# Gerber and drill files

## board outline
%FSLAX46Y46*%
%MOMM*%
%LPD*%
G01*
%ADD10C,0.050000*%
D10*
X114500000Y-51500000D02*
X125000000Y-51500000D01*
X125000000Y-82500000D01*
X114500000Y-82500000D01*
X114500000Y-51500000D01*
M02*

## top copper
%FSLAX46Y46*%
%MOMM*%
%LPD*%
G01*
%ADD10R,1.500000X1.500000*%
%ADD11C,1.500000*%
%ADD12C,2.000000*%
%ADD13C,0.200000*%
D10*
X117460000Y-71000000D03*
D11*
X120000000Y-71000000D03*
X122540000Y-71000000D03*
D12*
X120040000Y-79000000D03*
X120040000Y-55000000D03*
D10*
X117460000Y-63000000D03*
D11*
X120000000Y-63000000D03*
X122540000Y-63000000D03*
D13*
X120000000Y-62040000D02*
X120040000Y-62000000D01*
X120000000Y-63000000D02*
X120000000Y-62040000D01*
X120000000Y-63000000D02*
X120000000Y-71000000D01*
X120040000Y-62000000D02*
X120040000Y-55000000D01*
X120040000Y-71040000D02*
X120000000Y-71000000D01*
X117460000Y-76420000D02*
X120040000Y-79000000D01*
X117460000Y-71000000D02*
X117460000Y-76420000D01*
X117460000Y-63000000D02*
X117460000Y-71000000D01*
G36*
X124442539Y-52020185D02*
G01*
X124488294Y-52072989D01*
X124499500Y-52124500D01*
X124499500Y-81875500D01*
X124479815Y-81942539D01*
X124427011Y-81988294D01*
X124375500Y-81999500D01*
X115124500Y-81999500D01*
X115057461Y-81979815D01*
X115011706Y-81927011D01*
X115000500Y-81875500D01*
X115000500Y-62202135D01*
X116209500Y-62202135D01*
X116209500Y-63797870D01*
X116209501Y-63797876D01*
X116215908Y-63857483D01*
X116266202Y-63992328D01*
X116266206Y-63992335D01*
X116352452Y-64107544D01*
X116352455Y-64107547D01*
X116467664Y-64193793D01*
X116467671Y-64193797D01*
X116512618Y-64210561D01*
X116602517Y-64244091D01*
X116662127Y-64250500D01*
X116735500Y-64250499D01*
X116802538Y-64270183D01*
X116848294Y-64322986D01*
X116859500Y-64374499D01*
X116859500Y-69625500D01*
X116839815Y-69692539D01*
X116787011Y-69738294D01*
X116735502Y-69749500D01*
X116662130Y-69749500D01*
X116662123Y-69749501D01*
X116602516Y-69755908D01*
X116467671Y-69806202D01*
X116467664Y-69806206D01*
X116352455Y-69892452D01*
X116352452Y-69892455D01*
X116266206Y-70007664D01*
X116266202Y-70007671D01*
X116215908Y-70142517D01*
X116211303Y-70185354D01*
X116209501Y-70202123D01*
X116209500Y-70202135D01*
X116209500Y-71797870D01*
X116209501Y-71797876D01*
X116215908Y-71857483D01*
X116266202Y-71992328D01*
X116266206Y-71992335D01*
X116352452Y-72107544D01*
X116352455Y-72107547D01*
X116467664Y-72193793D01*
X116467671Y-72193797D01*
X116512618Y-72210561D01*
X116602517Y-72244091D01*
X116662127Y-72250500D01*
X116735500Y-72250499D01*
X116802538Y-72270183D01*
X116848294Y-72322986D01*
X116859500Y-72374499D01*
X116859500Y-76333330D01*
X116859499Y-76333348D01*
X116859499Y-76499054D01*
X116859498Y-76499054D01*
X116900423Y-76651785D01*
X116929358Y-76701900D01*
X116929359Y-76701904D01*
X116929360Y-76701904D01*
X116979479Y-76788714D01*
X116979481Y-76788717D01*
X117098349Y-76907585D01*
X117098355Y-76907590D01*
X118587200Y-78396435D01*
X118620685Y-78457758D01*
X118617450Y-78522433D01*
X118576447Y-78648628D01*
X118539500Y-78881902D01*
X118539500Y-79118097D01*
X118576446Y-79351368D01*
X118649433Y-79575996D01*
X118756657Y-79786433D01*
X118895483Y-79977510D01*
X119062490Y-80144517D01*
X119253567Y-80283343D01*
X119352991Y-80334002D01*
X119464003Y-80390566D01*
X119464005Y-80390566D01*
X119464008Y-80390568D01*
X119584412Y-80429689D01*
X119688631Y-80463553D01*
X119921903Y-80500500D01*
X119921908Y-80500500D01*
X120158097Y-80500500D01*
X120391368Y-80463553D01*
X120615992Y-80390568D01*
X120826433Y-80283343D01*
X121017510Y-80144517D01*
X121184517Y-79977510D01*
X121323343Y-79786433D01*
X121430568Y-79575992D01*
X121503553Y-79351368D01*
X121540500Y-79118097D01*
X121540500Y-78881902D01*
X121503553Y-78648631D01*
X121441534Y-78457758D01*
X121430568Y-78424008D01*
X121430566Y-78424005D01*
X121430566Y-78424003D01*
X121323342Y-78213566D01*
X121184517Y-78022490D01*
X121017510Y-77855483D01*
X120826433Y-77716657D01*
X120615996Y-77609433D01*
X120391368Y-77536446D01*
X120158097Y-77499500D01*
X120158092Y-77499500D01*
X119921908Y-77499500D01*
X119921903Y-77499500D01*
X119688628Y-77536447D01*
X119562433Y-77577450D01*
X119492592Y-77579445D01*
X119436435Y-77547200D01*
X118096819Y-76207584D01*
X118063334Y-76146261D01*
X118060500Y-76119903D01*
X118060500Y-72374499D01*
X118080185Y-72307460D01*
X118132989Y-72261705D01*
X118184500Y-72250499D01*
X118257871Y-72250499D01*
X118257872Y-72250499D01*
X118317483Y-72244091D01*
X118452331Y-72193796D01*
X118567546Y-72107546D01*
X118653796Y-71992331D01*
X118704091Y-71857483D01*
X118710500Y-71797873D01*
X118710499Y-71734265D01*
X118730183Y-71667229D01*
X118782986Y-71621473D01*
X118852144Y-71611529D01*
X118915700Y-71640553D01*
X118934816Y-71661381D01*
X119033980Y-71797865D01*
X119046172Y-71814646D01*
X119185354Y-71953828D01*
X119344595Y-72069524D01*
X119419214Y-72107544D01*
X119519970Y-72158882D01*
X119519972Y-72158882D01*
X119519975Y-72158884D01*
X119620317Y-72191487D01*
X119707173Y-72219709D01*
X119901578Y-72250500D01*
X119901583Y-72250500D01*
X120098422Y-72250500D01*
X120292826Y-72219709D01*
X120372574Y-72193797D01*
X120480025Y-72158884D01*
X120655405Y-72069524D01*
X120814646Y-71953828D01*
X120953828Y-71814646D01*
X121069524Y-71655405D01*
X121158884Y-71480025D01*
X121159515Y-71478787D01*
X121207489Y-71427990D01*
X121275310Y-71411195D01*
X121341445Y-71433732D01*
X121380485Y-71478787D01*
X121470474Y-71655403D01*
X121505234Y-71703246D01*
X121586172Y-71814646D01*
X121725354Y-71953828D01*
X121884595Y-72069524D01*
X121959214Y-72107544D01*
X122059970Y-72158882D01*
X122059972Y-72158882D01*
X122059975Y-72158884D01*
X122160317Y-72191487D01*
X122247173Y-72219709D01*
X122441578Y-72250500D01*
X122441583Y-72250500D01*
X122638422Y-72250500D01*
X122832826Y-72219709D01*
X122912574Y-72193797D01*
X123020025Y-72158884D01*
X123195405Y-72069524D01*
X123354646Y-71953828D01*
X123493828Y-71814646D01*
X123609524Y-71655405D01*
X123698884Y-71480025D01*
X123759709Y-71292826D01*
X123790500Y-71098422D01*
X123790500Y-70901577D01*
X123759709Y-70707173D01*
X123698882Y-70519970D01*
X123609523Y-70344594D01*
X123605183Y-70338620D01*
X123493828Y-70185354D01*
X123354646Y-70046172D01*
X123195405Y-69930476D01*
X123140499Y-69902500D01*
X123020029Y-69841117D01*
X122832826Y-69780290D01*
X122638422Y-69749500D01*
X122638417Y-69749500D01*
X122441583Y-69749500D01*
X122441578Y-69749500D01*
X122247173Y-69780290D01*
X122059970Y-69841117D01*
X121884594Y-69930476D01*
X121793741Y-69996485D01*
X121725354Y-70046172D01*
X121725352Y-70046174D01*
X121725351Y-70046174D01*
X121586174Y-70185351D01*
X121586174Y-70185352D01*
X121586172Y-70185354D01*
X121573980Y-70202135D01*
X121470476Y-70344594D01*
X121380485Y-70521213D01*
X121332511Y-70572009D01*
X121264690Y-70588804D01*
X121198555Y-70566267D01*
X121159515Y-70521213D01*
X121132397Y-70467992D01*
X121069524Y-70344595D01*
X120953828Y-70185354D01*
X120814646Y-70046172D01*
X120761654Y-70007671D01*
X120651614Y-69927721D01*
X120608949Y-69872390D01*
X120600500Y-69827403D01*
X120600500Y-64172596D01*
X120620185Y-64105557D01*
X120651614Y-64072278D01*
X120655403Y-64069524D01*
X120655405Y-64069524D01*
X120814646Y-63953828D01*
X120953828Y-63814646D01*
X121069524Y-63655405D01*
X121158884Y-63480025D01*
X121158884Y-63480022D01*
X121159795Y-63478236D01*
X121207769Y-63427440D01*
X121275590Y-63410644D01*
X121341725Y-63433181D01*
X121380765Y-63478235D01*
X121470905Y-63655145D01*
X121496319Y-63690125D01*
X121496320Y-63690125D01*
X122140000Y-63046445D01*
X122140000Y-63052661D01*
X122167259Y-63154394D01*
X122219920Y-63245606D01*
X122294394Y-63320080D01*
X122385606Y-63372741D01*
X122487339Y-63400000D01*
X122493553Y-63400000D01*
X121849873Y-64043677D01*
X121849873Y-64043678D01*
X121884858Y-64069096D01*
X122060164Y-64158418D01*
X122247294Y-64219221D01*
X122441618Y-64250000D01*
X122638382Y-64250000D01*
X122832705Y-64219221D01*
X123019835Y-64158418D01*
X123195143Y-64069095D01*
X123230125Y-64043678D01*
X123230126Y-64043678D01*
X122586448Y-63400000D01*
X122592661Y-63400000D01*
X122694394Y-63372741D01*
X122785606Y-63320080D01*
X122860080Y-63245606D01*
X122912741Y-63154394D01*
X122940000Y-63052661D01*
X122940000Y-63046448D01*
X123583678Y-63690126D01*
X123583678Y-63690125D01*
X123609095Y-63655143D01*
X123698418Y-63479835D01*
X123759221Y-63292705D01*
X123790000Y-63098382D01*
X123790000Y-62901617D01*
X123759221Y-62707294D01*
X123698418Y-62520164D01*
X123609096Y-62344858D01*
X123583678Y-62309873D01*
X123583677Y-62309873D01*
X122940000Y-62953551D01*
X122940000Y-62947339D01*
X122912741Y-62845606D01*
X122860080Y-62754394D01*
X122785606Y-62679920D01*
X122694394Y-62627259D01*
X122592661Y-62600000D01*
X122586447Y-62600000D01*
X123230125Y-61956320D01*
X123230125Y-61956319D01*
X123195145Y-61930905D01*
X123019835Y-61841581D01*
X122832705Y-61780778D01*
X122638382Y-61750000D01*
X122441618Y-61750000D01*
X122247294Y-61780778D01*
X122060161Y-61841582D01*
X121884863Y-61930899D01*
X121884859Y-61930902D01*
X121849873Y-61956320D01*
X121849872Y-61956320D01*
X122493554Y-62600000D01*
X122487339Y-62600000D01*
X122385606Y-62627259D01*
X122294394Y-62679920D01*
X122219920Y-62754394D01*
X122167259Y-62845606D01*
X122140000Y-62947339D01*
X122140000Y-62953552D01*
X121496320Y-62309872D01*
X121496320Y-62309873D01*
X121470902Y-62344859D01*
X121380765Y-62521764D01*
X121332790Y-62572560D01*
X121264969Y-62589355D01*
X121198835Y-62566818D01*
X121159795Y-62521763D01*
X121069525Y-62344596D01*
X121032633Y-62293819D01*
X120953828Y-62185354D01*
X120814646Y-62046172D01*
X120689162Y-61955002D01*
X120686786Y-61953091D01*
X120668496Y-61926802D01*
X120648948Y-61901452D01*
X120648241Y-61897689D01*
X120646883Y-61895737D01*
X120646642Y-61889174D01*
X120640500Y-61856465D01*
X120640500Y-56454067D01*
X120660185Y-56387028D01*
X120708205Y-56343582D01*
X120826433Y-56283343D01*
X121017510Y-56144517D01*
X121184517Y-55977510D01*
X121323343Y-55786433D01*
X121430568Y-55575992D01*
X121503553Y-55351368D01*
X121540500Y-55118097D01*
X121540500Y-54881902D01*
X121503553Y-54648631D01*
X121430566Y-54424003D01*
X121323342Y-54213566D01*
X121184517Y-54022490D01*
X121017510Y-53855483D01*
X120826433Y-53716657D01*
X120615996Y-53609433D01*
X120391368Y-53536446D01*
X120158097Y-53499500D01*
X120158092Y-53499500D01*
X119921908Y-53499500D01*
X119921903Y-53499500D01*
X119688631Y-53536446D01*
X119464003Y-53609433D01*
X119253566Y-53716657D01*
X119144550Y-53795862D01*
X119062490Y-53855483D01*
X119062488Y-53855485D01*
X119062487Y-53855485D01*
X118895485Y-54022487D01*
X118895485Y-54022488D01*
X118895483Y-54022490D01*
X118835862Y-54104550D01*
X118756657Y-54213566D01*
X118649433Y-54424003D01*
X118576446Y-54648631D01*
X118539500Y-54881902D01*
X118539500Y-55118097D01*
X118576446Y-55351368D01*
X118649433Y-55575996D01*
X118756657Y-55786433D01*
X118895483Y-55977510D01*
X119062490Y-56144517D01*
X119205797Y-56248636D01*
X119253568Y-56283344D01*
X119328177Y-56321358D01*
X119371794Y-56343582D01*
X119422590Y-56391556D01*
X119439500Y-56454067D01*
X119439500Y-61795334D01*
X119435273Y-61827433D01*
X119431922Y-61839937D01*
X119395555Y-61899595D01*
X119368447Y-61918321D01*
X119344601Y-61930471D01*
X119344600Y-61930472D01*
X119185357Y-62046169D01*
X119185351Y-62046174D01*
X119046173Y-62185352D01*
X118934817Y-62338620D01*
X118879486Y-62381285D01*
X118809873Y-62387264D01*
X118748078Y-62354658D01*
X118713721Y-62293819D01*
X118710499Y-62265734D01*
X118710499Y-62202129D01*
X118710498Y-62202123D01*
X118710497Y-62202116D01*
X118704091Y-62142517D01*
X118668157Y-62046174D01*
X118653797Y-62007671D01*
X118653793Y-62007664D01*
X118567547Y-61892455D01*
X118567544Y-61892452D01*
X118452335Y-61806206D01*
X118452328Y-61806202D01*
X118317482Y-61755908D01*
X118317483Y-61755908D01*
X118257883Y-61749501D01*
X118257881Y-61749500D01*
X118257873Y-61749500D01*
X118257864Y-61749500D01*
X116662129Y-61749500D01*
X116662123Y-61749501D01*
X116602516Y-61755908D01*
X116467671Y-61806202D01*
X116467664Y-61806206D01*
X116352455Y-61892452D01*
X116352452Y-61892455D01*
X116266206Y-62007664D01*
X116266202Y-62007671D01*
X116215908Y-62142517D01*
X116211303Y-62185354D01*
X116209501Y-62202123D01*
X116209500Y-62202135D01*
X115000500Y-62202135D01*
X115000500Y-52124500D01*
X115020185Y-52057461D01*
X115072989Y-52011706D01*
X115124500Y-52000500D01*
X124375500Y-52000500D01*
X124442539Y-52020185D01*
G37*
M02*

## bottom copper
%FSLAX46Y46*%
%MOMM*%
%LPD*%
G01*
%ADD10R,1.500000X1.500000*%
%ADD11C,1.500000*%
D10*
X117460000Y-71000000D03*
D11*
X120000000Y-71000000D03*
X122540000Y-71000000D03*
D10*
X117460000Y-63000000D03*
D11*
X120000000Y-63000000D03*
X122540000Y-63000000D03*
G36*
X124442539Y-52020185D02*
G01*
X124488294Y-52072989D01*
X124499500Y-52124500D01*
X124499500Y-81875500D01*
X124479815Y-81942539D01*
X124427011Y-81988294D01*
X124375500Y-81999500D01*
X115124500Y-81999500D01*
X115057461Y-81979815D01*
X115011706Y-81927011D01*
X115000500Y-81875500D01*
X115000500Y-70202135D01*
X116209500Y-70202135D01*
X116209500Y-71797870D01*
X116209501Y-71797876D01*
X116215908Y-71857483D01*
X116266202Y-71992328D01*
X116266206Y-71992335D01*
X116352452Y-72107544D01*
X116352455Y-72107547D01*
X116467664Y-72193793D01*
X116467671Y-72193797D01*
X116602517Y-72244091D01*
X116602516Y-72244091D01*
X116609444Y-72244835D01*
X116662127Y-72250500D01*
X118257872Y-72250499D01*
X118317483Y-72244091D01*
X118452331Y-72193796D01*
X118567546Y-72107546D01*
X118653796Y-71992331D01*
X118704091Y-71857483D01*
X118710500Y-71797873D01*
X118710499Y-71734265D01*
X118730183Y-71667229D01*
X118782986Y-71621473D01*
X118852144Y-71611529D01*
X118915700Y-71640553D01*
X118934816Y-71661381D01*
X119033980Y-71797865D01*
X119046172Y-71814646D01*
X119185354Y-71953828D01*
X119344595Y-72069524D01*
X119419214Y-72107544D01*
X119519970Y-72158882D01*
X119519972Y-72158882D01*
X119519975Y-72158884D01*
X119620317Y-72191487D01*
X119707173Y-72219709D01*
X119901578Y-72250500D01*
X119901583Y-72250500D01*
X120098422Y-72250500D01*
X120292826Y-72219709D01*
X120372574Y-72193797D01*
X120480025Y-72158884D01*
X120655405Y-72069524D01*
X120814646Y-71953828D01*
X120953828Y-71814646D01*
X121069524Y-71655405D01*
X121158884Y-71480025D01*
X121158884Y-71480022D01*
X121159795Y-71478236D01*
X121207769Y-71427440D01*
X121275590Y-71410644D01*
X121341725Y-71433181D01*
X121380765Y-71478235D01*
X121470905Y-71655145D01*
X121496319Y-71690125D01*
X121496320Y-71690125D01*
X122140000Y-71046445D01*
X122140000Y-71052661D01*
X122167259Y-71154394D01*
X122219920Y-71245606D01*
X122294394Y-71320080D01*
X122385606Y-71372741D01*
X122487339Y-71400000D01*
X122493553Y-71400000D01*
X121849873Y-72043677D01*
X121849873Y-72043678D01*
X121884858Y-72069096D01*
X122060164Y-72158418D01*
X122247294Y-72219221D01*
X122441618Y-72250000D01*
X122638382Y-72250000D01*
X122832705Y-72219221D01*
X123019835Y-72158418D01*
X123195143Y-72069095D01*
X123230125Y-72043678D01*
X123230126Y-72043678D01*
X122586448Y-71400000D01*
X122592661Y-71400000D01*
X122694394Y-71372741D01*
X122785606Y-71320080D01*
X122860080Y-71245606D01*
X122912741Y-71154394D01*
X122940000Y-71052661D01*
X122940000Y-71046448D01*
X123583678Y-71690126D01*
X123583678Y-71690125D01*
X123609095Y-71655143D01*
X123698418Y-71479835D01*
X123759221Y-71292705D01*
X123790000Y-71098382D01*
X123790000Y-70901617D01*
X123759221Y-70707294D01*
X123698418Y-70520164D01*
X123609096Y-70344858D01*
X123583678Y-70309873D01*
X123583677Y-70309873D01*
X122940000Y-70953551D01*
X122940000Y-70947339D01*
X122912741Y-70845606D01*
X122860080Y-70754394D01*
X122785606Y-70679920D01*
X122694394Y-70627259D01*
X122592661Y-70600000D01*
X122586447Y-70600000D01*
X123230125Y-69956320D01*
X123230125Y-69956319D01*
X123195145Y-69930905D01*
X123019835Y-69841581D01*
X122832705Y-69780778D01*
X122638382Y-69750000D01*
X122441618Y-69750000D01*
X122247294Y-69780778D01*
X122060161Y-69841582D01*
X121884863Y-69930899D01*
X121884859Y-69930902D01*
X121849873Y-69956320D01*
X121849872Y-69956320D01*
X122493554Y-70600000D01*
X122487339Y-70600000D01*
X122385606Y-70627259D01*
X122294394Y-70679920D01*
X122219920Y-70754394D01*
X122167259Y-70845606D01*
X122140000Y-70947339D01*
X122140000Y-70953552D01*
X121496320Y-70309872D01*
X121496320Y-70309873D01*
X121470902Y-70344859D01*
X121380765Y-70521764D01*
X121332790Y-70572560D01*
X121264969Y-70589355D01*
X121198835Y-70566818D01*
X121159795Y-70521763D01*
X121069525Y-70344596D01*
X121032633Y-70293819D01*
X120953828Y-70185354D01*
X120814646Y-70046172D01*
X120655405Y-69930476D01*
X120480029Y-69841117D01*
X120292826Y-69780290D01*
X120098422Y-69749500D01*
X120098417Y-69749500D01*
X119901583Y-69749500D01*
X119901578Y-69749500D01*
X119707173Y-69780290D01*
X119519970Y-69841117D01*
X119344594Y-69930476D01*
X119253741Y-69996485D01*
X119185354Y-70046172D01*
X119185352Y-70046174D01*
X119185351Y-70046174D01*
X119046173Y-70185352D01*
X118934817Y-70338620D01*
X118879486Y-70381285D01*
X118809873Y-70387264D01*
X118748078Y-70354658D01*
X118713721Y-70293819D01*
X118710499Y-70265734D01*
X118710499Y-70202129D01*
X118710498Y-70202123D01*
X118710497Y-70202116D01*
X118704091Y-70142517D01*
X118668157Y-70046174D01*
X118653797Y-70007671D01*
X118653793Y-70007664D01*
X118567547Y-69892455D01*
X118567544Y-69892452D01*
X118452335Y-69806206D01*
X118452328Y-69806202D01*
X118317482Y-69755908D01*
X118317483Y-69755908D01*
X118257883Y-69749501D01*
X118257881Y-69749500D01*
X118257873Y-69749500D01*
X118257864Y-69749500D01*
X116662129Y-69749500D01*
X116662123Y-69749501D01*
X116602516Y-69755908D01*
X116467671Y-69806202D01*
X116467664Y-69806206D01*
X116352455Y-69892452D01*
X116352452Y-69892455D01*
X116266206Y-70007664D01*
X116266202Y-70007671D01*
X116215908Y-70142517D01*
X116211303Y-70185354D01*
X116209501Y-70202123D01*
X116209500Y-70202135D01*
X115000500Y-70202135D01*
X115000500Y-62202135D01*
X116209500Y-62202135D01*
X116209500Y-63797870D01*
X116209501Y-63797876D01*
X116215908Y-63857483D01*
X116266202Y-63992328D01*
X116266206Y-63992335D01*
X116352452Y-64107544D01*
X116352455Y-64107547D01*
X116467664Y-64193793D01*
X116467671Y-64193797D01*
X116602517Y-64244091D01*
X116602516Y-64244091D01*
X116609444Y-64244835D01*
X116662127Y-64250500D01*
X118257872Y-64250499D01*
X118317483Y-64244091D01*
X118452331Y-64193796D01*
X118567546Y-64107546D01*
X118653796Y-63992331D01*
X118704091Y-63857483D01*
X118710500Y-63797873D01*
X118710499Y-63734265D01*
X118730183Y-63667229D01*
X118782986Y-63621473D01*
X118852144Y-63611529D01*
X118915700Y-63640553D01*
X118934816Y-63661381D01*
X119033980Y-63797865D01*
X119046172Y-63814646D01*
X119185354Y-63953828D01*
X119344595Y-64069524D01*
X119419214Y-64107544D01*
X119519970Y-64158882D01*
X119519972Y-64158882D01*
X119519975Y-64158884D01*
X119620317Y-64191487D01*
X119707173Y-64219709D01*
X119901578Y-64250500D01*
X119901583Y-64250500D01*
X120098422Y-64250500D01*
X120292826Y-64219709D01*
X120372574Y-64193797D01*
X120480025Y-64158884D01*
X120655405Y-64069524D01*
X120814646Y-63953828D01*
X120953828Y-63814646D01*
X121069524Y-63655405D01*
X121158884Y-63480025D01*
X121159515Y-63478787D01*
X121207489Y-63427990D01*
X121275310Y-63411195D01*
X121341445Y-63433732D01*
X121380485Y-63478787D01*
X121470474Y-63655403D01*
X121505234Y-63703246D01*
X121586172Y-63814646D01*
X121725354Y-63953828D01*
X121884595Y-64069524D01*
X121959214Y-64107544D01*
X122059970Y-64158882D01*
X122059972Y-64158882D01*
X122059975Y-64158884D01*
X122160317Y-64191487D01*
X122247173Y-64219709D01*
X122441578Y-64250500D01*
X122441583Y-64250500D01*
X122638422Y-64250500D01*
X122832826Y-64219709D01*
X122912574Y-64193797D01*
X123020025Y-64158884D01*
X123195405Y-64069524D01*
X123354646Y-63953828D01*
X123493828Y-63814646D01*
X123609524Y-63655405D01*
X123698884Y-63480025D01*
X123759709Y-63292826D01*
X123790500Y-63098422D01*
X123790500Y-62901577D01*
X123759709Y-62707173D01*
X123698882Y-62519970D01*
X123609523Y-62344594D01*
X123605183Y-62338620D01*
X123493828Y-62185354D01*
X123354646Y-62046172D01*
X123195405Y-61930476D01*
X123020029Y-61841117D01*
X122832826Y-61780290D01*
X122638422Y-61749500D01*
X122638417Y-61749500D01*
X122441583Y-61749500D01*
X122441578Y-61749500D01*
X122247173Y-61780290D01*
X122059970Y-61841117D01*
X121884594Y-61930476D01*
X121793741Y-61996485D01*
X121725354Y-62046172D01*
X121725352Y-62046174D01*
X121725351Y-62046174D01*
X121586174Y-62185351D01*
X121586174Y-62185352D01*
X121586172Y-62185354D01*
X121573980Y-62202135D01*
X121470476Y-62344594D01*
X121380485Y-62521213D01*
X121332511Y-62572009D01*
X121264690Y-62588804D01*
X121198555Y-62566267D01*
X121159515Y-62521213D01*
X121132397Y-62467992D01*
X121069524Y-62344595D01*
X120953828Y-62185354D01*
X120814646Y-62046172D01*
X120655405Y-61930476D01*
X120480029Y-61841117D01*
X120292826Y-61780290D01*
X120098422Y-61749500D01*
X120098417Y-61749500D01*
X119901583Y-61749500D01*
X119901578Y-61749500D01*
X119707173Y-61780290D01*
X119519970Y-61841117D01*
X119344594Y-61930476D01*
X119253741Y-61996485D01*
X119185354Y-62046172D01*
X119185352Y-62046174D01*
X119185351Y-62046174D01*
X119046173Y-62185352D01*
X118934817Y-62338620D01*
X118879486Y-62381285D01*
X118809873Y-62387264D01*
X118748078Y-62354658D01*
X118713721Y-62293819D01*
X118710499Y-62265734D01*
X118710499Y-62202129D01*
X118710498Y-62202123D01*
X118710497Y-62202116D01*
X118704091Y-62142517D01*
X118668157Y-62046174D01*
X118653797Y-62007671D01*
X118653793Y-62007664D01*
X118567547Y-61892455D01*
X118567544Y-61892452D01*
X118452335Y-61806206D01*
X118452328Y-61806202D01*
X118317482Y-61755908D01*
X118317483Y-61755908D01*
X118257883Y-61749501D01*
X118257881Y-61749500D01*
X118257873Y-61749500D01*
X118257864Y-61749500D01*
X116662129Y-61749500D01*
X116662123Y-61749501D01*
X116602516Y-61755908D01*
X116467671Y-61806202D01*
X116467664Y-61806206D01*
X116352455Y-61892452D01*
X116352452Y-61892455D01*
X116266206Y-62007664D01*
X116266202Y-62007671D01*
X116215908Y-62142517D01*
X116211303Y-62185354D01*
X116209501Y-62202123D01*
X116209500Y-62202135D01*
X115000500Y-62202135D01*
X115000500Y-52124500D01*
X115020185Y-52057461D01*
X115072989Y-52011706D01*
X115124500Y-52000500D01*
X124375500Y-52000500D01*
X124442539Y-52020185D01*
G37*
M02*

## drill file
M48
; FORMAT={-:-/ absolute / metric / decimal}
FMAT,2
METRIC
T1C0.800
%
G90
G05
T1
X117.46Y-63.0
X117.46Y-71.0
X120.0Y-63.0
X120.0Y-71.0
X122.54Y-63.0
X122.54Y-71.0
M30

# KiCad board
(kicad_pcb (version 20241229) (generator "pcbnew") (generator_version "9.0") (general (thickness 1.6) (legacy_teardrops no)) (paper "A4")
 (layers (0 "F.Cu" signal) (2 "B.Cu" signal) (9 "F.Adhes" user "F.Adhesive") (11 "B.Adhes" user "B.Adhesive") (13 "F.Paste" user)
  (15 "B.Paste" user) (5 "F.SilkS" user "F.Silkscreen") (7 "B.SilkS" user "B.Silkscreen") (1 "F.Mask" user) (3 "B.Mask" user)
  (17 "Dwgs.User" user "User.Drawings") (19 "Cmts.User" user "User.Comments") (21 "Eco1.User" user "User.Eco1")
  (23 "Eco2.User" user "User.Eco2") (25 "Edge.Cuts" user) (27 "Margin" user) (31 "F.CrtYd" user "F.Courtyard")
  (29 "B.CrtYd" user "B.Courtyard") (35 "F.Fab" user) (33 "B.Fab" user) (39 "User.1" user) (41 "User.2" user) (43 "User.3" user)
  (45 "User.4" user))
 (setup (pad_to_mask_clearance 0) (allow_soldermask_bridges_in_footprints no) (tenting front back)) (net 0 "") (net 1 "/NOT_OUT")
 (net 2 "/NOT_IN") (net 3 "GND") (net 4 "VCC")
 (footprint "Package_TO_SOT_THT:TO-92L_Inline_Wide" (layer "F.Cu") (at 117.46 71)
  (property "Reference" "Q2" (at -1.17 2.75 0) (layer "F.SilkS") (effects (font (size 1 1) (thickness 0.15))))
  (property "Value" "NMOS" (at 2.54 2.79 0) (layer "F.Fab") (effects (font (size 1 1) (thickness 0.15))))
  (pad "1" thru_hole rect (at 0 0) (size 1.5 1.5) (drill 0.8) (layers "*.Cu" "*.Mask") (remove_unused_layers no) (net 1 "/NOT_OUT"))
  (pad "2" thru_hole circle (at 2.54 0) (size 1.5 1.5) (drill 0.8) (layers "*.Cu" "*.Mask") (remove_unused_layers no) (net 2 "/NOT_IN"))
  (pad "3" thru_hole circle (at 5.08 0) (size 1.5 1.5) (drill 0.8) (layers "*.Cu" "*.Mask") (remove_unused_layers no) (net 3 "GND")))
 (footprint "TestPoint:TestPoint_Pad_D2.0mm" (layer "F.Cu") (at 120.04 79)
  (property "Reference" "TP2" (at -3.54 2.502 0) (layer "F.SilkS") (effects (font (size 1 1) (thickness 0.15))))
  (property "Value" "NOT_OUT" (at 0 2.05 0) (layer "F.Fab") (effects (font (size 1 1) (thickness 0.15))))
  (pad "1" smd circle (at 0 0) (size 2 2) (layers "F.Cu" "F.Mask") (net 1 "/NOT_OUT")))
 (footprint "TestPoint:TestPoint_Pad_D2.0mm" (layer "F.Cu") (at 120.04 55)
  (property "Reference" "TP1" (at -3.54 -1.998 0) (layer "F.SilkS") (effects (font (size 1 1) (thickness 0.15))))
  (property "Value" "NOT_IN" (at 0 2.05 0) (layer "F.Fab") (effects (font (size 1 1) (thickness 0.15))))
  (pad "1" smd circle (at 0 0) (size 2 2) (layers "F.Cu" "F.Mask") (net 2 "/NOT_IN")))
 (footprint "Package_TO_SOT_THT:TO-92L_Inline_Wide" (layer "F.Cu") (at 117.46 63)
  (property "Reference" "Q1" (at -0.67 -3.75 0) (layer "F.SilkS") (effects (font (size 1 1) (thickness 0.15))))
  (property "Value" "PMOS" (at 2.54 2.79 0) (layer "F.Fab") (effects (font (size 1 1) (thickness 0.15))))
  (pad "1" thru_hole rect (at 0 0) (size 1.5 1.5) (drill 0.8) (layers "*.Cu" "*.Mask") (remove_unused_layers no) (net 1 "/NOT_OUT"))
  (pad "2" thru_hole circle (at 2.54 0) (size 1.5 1.5) (drill 0.8) (layers "*.Cu" "*.Mask") (remove_unused_layers no) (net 2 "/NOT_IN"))
  (pad "3" thru_hole circle (at 5.08 0) (size 1.5 1.5) (drill 0.8) (layers "*.Cu" "*.Mask") (remove_unused_layers no) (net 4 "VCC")))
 (gr_rect (start 114.5 51.5) (end 125 82.5) (stroke (width 0.05) (type default)) (fill no) (layer "Edge.Cuts"))
 (segment (start 120 62.04) (end 120.04 62) (width 0.2) (layer "F.Cu") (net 2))
 (segment (start 120 63) (end 120 62.04) (width 0.2) (layer "F.Cu") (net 2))
 (segment (start 120 63) (end 120 71) (width 0.2) (layer "F.Cu") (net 2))
 (segment (start 120.04 62) (end 120.04 55) (width 0.2) (layer "F.Cu") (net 2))
 (segment (start 120.04 71.04) (end 120 71) (width 0.2) (layer "F.Cu") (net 2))
 (segment (start 117.46 76.42) (end 120.04 79) (width 0.2) (layer "F.Cu") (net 1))
 (segment (start 117.46 71) (end 117.46 76.42) (width 0.2) (layer "F.Cu") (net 1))
 (segment (start 117.46 63) (end 117.46 71) (width 0.2) (layer "F.Cu") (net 1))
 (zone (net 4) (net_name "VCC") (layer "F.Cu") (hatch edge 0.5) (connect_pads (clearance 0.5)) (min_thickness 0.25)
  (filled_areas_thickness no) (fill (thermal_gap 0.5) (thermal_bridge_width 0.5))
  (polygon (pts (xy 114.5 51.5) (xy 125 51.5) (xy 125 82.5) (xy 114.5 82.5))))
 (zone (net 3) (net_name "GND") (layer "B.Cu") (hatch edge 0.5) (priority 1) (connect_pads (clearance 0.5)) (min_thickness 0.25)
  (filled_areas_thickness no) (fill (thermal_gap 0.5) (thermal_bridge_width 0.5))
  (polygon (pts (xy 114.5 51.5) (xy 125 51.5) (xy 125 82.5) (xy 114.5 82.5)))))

